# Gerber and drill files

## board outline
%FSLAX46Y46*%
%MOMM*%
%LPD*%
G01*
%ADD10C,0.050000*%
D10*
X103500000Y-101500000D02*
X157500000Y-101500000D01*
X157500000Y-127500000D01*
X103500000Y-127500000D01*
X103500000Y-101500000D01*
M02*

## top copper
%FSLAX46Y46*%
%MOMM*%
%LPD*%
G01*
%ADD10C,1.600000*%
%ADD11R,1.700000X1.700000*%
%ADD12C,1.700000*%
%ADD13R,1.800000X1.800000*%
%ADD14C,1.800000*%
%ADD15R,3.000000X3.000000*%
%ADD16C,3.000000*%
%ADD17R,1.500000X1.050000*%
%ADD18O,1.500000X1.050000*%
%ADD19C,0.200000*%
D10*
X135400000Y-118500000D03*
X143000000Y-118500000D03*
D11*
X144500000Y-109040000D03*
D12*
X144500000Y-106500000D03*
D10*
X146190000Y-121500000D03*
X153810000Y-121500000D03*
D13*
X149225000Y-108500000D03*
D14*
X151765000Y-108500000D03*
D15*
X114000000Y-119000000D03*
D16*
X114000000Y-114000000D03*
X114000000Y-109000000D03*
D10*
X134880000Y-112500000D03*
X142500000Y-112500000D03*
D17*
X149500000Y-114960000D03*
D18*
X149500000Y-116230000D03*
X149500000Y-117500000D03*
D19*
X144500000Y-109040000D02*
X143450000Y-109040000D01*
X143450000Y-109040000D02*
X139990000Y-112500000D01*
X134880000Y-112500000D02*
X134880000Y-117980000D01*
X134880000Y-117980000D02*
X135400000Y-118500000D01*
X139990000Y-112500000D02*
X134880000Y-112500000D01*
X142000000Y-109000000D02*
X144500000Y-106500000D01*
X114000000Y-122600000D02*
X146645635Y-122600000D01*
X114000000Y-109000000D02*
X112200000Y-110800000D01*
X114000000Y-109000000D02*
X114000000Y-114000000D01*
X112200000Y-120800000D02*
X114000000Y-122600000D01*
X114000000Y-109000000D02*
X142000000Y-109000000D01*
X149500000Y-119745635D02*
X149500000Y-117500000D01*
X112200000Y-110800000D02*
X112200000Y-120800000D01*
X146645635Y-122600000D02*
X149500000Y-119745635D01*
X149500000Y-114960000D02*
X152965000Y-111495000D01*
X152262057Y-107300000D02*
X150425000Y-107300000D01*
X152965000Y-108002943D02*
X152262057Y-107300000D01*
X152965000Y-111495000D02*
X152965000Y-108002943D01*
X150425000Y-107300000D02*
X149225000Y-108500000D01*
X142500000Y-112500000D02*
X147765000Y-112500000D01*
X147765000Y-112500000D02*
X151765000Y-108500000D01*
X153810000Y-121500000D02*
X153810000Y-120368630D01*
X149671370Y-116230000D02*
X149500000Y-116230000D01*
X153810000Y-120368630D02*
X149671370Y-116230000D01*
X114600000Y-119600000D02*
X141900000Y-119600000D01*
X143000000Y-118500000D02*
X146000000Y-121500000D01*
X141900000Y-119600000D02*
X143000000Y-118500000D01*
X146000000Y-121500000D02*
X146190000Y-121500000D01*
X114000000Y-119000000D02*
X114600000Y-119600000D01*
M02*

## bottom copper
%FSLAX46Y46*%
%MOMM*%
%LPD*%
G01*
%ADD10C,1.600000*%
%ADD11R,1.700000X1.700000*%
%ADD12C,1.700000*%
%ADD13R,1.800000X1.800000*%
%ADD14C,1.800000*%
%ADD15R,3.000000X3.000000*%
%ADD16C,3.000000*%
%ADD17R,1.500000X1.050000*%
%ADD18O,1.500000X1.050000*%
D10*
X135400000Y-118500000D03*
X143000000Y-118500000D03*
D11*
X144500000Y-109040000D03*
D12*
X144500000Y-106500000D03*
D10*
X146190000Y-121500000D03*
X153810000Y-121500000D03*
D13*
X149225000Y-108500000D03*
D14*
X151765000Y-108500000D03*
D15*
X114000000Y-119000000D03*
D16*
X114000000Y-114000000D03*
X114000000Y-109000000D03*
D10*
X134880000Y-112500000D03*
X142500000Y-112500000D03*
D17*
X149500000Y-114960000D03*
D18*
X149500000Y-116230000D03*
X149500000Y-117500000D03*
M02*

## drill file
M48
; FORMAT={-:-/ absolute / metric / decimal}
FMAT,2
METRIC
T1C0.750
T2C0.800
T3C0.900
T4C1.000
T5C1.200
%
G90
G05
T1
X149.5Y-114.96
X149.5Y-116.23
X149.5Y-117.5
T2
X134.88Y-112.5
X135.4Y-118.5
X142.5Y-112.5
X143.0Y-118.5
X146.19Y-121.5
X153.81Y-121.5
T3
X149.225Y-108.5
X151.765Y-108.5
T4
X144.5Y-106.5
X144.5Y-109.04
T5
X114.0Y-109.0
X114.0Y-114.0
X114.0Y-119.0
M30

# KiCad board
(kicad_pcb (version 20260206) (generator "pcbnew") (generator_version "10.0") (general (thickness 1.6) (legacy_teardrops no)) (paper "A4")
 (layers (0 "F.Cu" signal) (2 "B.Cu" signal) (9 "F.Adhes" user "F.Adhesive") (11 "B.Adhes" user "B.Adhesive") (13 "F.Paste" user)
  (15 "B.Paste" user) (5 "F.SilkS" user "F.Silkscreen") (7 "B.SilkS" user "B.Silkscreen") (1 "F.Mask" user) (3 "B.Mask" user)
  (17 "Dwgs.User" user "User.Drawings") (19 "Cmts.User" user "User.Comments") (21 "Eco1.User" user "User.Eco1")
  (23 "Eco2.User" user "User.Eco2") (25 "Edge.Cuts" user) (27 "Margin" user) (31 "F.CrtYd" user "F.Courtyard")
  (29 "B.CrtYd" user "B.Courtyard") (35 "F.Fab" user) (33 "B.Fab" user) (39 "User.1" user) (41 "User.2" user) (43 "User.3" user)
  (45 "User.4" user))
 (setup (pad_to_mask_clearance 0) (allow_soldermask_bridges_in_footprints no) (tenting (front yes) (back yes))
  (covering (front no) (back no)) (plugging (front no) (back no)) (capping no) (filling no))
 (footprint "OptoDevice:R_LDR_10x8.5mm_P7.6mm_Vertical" (layer "F.Cu") (at 135.4 118.5)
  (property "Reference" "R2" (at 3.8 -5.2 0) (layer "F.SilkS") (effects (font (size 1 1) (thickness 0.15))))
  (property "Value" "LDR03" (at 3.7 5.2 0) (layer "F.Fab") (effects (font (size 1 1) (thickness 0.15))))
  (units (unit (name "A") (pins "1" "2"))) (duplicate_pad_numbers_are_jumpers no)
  (pad "1" thru_hole circle (at 0 0) (size 1.6 1.6) (drill 0.8) (layers "*.Cu" "*.Mask") (remove_unused_layers no) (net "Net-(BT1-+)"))
  (pad "2" thru_hole circle (at 7.6 0) (size 1.6 1.6) (drill 0.8) (layers "*.Cu" "*.Mask") (remove_unused_layers no) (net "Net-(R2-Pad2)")))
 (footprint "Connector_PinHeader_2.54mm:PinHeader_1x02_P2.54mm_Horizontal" (layer "F.Cu") (at 144.5 109.04 180)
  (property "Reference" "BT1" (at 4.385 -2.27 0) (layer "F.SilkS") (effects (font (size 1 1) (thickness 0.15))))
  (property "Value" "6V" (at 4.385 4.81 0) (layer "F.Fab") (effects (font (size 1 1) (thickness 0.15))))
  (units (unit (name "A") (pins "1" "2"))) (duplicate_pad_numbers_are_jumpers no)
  (pad "1" thru_hole rect (at 0 0 180) (size 1.7 1.7) (drill 1) (layers "*.Cu" "*.Mask") (remove_unused_layers no) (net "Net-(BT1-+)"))
  (pad "2" thru_hole circle (at 0 2.54 180) (size 1.7 1.7) (drill 1) (layers "*.Cu" "*.Mask") (remove_unused_layers no) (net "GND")))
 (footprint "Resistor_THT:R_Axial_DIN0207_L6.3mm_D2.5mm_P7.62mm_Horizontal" (layer "F.Cu") (at 146.19 121.5)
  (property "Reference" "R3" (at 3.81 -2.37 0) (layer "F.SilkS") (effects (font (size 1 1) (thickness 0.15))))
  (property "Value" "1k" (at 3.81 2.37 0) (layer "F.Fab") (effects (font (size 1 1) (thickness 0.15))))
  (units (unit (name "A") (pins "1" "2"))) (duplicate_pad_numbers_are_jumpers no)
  (pad "1" thru_hole circle (at 0 0) (size 1.6 1.6) (drill 0.8) (layers "*.Cu" "*.Mask") (remove_unused_layers no) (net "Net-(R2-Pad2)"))
  (pad "2" thru_hole circle (at 7.62 0) (size 1.6 1.6) (drill 0.8) (layers "*.Cu" "*.Mask") (remove_unused_layers no) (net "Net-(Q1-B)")))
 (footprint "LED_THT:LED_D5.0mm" (layer "F.Cu") (at 149.225 108.5)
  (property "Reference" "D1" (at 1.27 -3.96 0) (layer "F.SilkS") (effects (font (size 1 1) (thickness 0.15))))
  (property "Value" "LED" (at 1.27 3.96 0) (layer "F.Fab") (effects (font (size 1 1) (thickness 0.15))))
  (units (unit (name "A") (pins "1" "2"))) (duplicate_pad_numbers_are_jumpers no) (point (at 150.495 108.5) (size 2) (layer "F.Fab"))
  (pad "1" thru_hole rect (at 0 0) (size 1.8 1.8) (drill 0.9) (layers "*.Cu" "*.Mask") (remove_unused_layers no) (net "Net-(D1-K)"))
  (pad "2" thru_hole circle (at 2.54 0) (size 1.8 1.8) (drill 0.9) (layers "*.Cu" "*.Mask") (remove_unused_layers no) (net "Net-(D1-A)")))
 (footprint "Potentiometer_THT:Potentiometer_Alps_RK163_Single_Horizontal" (layer "F.Cu") (at 114 119 180)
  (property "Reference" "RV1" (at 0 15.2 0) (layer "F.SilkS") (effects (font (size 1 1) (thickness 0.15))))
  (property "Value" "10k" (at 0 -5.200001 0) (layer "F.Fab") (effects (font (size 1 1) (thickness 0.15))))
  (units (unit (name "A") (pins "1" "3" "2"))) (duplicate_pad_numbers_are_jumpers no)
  (pad "1" thru_hole rect (at 0 0) (size 3 3) (drill 1.2) (layers "*.Cu" "*.Mask") (remove_unused_layers no) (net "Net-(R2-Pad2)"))
  (pad "2" thru_hole circle (at 0 5) (size 3 3) (drill 1.2) (layers "*.Cu" "*.Mask") (remove_unused_layers no) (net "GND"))
  (pad "3" thru_hole circle (at 0 10) (size 3 3) (drill 1.2) (layers "*.Cu" "*.Mask") (remove_unused_layers no) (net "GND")))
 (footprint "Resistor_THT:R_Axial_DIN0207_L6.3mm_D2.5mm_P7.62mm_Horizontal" (layer "F.Cu") (at 134.88 112.5)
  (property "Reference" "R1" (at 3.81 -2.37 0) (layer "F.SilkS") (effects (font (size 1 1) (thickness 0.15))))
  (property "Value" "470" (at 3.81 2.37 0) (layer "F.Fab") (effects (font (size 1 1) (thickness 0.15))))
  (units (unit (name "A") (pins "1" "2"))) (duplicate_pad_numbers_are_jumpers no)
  (pad "1" thru_hole circle (at 0 0) (size 1.6 1.6) (drill 0.8) (layers "*.Cu" "*.Mask") (remove_unused_layers no) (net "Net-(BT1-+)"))
  (pad "2" thru_hole circle (at 7.62 0) (size 1.6 1.6) (drill 0.8) (layers "*.Cu" "*.Mask") (remove_unused_layers no) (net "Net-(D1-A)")))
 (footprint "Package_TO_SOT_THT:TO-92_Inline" (layer "F.Cu") (at 149.5 114.96 -90)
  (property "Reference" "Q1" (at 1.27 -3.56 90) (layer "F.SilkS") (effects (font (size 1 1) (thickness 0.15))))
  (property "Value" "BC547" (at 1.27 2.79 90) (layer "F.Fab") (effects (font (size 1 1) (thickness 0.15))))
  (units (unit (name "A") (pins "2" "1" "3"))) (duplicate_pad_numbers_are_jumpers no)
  (pad "1" thru_hole rect (at 0 0 270) (size 1.05 1.5) (drill 0.75) (layers "*.Cu" "*.Mask") (remove_unused_layers no) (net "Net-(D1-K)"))
  (pad "2" thru_hole oval (at 1.27 0 270) (size 1.05 1.5) (drill 0.75) (layers "*.Cu" "*.Mask") (remove_unused_layers no) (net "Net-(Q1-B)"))
  (pad "3" thru_hole oval (at 2.54 0 270) (size 1.05 1.5) (drill 0.75) (layers "*.Cu" "*.Mask") (remove_unused_layers no) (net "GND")))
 (gr_rect (start 103.5 101.5) (end 157.5 127.5) (stroke (width 0.05) (type default)) (fill no) (layer "Edge.Cuts"))
 (segment (start 144.5 109.04) (end 143.45 109.04) (width 0.2) (layer "F.Cu") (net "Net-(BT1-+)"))
 (segment (start 143.45 109.04) (end 139.99 112.5) (width 0.2) (layer "F.Cu") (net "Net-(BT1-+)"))
 (segment (start 134.88 112.5) (end 134.88 117.98) (width 0.2) (layer "F.Cu") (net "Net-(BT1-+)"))
 (segment (start 134.88 117.98) (end 135.4 118.5) (width 0.2) (layer "F.Cu") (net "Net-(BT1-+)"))
 (segment (start 139.99 112.5) (end 134.88 112.5) (width 0.2) (layer "F.Cu") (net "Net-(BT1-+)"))
 (segment (start 142 109) (end 144.5 106.5) (width 0.2) (layer "F.Cu") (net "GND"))
 (segment (start 114 122.6) (end 146.645635 122.6) (width 0.2) (layer "F.Cu") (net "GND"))
 (segment (start 114 109) (end 112.2 110.8) (width 0.2) (layer "F.Cu") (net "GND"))
 (segment (start 114 109) (end 114 114) (width 0.2) (layer "F.Cu") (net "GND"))
 (segment (start 112.2 120.8) (end 114 122.6) (width 0.2) (layer "F.Cu") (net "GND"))
 (segment (start 114 109) (end 142 109) (width 0.2) (layer "F.Cu") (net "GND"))
 (segment (start 149.5 119.745635) (end 149.5 117.5) (width 0.2) (layer "F.Cu") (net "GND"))
 (segment (start 112.2 110.8) (end 112.2 120.8) (width 0.2) (layer "F.Cu") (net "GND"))
 (segment (start 146.645635 122.6) (end 149.5 119.745635) (width 0.2) (layer "F.Cu") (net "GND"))
 (segment (start 149.5 114.96) (end 152.965 111.495) (width 0.2) (layer "F.Cu") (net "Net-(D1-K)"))
 (segment (start 152.262057 107.3) (end 150.425 107.3) (width 0.2) (layer "F.Cu") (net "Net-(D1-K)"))
 (segment (start 152.965 108.002943) (end 152.262057 107.3) (width 0.2) (layer "F.Cu") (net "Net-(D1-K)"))
 (segment (start 152.965 111.495) (end 152.965 108.002943) (width 0.2) (layer "F.Cu") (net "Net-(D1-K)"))
 (segment (start 150.425 107.3) (end 149.225 108.5) (width 0.2) (layer "F.Cu") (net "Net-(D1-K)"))
 (segment (start 142.5 112.5) (end 147.765 112.5) (width 0.2) (layer "F.Cu") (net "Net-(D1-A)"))
 (segment (start 147.765 112.5) (end 151.765 108.5) (width 0.2) (layer "F.Cu") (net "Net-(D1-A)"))
 (segment (start 153.81 121.5) (end 153.81 120.36863) (width 0.2) (layer "F.Cu") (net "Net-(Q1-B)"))
 (segment (start 149.67137 116.23) (end 149.5 116.23) (width 0.2) (layer "F.Cu") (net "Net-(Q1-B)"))
 (segment (start 153.81 120.36863) (end 149.67137 116.23) (width 0.2) (layer "F.Cu") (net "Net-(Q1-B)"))
 (segment (start 114.6 119.6) (end 141.9 119.6) (width 0.2) (layer "F.Cu") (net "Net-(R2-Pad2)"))
 (segment (start 143 118.5) (end 146 121.5) (width 0.2) (layer "F.Cu") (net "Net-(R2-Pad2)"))
 (segment (start 141.9 119.6) (end 143 118.5) (width 0.2) (layer "F.Cu") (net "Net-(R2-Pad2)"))
 (segment (start 146 121.5) (end 146.19 121.5) (width 0.2) (layer "F.Cu") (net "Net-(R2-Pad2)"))
 (segment (start 114 119) (end 114.6 119.6) (width 0.2) (layer "F.Cu") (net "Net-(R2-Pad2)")))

